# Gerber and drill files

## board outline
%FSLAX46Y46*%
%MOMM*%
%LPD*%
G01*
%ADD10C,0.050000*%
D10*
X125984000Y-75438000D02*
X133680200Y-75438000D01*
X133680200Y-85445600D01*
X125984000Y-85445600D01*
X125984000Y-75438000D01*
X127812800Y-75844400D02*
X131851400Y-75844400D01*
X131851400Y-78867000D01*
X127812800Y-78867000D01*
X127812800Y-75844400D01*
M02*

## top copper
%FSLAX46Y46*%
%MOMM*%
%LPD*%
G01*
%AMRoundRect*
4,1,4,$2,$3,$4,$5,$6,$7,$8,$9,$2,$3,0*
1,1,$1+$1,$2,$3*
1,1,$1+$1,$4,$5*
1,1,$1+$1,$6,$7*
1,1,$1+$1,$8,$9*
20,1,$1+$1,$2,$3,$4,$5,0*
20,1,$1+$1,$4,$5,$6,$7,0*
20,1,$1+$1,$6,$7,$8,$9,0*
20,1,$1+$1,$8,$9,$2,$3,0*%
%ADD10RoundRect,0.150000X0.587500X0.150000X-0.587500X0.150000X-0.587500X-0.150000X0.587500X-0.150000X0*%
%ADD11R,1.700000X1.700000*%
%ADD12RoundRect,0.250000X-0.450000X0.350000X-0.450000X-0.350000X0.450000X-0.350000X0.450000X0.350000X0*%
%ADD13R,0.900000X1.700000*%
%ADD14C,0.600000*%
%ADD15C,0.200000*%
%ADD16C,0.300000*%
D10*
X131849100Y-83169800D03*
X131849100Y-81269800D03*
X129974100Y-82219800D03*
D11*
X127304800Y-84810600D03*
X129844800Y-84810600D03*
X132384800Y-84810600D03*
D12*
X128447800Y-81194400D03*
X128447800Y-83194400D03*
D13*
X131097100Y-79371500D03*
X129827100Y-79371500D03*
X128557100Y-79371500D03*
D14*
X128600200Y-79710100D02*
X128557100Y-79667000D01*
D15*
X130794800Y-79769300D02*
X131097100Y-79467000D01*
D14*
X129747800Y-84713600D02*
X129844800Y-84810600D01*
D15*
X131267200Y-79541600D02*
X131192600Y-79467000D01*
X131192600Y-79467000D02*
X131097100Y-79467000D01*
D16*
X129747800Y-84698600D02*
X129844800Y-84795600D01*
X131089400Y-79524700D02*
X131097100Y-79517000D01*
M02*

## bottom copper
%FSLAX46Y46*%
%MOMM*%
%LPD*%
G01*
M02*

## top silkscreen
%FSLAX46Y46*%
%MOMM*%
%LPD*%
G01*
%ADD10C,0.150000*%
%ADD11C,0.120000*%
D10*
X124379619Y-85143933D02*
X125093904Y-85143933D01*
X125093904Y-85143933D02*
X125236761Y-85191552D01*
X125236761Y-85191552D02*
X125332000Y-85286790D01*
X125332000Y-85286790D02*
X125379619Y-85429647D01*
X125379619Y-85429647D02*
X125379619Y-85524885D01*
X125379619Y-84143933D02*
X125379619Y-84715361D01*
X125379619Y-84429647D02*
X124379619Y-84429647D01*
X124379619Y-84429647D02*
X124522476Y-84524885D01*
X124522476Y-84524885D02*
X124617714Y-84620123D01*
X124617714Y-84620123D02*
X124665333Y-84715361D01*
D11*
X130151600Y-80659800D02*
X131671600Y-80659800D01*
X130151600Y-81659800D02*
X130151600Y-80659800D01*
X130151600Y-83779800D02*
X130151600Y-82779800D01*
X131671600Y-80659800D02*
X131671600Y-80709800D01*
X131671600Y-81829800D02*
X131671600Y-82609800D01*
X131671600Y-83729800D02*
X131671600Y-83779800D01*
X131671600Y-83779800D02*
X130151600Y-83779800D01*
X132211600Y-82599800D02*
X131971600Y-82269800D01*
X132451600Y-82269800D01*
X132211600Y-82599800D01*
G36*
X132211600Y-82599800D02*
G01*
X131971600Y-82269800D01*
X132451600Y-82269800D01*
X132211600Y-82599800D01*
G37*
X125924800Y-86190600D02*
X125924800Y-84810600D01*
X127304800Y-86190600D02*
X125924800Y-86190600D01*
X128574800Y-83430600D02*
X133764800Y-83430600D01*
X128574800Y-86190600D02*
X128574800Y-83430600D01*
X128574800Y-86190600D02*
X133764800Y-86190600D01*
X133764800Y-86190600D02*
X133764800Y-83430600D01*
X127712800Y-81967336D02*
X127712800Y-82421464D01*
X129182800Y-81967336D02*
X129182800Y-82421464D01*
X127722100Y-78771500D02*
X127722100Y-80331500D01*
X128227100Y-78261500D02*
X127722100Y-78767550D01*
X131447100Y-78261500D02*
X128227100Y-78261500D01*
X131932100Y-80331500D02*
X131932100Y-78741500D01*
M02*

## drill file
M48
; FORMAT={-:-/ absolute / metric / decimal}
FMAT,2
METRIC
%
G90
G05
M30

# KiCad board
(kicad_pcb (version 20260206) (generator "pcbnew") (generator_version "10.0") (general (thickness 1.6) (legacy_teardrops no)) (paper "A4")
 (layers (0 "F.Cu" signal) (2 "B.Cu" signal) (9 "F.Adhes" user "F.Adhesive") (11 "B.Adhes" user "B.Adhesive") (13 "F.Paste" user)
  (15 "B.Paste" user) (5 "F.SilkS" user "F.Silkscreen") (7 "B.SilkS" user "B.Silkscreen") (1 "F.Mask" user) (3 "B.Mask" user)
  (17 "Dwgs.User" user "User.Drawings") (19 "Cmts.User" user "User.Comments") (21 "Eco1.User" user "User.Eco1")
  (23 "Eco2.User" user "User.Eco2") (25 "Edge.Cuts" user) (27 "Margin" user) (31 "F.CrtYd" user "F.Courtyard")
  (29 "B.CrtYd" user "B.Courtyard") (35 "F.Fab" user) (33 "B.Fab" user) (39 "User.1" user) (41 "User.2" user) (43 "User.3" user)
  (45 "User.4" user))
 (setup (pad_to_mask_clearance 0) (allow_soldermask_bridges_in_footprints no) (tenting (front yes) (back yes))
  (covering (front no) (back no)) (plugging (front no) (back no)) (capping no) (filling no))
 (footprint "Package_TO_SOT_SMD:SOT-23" (layer "F.Cu") (at 130.9116 82.2198 180)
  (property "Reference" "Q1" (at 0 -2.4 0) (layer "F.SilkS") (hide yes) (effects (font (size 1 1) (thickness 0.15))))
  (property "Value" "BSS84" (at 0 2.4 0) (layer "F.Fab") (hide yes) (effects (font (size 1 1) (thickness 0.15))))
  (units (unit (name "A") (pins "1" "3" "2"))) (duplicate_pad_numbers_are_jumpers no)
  (fp_line (start 0.76 1.56) (end -0.76 1.56) (stroke (width 0.12) (type solid)) (layer "F.SilkS"))
  (fp_line (start 0.76 0.56) (end 0.76 1.56) (stroke (width 0.12) (type solid)) (layer "F.SilkS"))
  (fp_line (start 0.76 -1.56) (end 0.76 -0.56) (stroke (width 0.12) (type solid)) (layer "F.SilkS"))
  (fp_line (start -0.76 1.56) (end -0.76 1.51) (stroke (width 0.12) (type solid)) (layer "F.SilkS"))
  (fp_line (start -0.76 0.39) (end -0.76 -0.39) (stroke (width 0.12) (type solid)) (layer "F.SilkS"))
  (fp_line (start -0.76 -1.51) (end -0.76 -1.56) (stroke (width 0.12) (type solid)) (layer "F.SilkS"))
  (fp_line (start -0.76 -1.56) (end 0.76 -1.56) (stroke (width 0.12) (type solid)) (layer "F.SilkS"))
  (fp_poly (pts (xy -1.3 -0.38) (xy -1.06 -0.05) (xy -1.54 -0.05)) (stroke (width 0.12) (type solid)) (fill yes) (layer "F.SilkS"))
  (pad "1" smd roundrect (at -0.9375 -0.95 180) (size 1.475 0.6) (layers "F.Cu" "F.Mask" "F.Paste") (roundrect_rratio 0.25)
   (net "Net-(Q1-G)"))
  (pad "2" smd roundrect (at -0.9375 0.95 180) (size 1.475 0.6) (layers "F.Cu" "F.Mask" "F.Paste") (roundrect_rratio 0.25)
   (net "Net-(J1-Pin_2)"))
  (pad "3" smd roundrect (at 0.9375 0 180) (size 1.475 0.6) (layers "F.Cu" "F.Mask" "F.Paste") (roundrect_rratio 0.25)
   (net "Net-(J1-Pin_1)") (die_length 2)))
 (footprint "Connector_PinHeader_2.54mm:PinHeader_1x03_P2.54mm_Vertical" (layer "F.Cu") (at 127.3048 84.8106 90)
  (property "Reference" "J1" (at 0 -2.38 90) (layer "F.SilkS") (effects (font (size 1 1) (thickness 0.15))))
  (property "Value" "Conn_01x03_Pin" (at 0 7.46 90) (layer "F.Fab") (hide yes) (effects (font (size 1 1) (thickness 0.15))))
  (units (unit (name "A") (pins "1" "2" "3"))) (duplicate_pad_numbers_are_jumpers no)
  (fp_line (start -1.38 -1.38) (end 0 -1.38) (stroke (width 0.12) (type solid)) (layer "F.SilkS"))
  (fp_line (start -1.38 0) (end -1.38 -1.38) (stroke (width 0.12) (type solid)) (layer "F.SilkS"))
  (fp_line (start 1.38 1.27) (end 1.38 6.46) (stroke (width 0.12) (type solid)) (layer "F.SilkS"))
  (fp_line (start -1.38 1.27) (end 1.38 1.27) (stroke (width 0.12) (type solid)) (layer "F.SilkS"))
  (fp_line (start -1.38 1.27) (end -1.38 6.46) (stroke (width 0.12) (type solid)) (layer "F.SilkS"))
  (fp_line (start -1.38 6.46) (end 1.38 6.46) (stroke (width 0.12) (type solid)) (layer "F.SilkS"))
  (pad "1" smd rect (at 0 0 90) (size 1.7 1.7) (layers "F.Cu" "F.Mask" "F.Paste") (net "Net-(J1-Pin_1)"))
  (pad "2" smd rect (at 0 2.54 90) (size 1.7 1.7) (layers "F.Cu" "F.Mask" "F.Paste") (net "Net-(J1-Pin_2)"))
  (pad "3" smd rect (at 0 5.08 90) (size 1.7 1.7) (layers "F.Cu" "F.Mask" "F.Paste") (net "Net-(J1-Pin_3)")))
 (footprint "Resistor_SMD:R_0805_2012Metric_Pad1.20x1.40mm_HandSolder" (layer "F.Cu") (at 128.4478 82.1944 -90)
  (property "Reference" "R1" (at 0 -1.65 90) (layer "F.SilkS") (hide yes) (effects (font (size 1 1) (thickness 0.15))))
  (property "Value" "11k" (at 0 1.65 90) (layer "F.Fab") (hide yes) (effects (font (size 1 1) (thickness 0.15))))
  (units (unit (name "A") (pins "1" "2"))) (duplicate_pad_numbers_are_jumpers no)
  (fp_line (start -0.227064 0.735) (end 0.227064 0.735) (stroke (width 0.12) (type solid)) (layer "F.SilkS"))
  (fp_line (start -0.227064 -0.735) (end 0.227064 -0.735) (stroke (width 0.12) (type solid)) (layer "F.SilkS"))
  (pad "1" smd roundrect (at -1 0 270) (size 1.2 1.4) (layers "F.Cu" "F.Mask" "F.Paste") (roundrect_rratio 0.208333) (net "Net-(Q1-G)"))
  (pad "2" smd roundrect (at 1 0 270) (size 1.2 1.4) (layers "F.Cu" "F.Mask" "F.Paste") (roundrect_rratio 0.208333) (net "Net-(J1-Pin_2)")))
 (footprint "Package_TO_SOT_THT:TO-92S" (layer "F.Cu") (at 131.0971 79.3715 180)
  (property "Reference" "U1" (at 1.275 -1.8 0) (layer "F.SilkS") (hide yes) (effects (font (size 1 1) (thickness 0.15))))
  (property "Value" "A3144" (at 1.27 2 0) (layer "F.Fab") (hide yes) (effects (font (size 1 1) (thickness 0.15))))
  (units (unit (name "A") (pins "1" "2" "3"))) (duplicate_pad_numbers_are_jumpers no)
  (fp_line (start 3.375 0.6) (end 3.375 -0.96) (stroke (width 0.12) (type solid)) (layer "F.SilkS"))
  (fp_line (start 2.87 1.11) (end 3.375 0.60395) (stroke (width 0.12) (type solid)) (layer "F.SilkS"))
  (fp_line (start -0.35 1.11) (end 2.87 1.11) (stroke (width 0.12) (type solid)) (layer "F.SilkS"))
  (fp_line (start -0.835 -0.96) (end -0.835 0.63) (stroke (width 0.12) (type solid)) (layer "F.SilkS"))
  (pad "1" smd rect (at 0 0) (size 0.9 1.7) (layers "F.Cu" "F.Mask" "F.Paste") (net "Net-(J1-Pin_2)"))
  (pad "2" smd rect (at 1.27 0) (size 0.9 1.7) (layers "F.Cu" "F.Mask" "F.Paste") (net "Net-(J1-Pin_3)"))
  (pad "3" smd rect (at 2.54 0) (size 0.9 1.7) (layers "F.Cu" "F.Mask" "F.Paste") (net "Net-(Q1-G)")))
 (gr_rect (start 125.984 75.438) (end 133.6802 85.4456) (stroke (width 0.05) (type default)) (fill no) (layer "Edge.Cuts"))
 (gr_rect (start 127.8128 75.8444) (end 131.8514 78.867) (stroke (width 0.05) (type default)) (fill no) (layer "Edge.Cuts"))
 (segment (start 128.6002 79.7101) (end 128.5571 79.667) (width 0.6) (layer "F.Cu") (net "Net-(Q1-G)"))
 (segment (start 130.7948 79.7693) (end 131.0971 79.467) (width 0.2) (layer "F.Cu") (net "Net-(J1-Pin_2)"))
 (segment (start 129.7478 84.7136) (end 129.8448 84.8106) (width 0.6) (layer "F.Cu") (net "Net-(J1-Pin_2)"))
 (segment (start 131.2672 79.5416) (end 131.1926 79.467) (width 0.2) (layer "F.Cu") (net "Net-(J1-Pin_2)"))
 (segment (start 131.1926 79.467) (end 131.0971 79.467) (width 0.2) (layer "F.Cu") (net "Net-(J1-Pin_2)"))
 (segment (start 129.7478 84.6986) (end 129.8448 84.7956) (width 0.3) (layer "F.Cu") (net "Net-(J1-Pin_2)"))
 (segment (start 131.0894 79.5247) (end 131.0971 79.517) (width 0.3) (layer "F.Cu") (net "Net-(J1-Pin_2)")))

